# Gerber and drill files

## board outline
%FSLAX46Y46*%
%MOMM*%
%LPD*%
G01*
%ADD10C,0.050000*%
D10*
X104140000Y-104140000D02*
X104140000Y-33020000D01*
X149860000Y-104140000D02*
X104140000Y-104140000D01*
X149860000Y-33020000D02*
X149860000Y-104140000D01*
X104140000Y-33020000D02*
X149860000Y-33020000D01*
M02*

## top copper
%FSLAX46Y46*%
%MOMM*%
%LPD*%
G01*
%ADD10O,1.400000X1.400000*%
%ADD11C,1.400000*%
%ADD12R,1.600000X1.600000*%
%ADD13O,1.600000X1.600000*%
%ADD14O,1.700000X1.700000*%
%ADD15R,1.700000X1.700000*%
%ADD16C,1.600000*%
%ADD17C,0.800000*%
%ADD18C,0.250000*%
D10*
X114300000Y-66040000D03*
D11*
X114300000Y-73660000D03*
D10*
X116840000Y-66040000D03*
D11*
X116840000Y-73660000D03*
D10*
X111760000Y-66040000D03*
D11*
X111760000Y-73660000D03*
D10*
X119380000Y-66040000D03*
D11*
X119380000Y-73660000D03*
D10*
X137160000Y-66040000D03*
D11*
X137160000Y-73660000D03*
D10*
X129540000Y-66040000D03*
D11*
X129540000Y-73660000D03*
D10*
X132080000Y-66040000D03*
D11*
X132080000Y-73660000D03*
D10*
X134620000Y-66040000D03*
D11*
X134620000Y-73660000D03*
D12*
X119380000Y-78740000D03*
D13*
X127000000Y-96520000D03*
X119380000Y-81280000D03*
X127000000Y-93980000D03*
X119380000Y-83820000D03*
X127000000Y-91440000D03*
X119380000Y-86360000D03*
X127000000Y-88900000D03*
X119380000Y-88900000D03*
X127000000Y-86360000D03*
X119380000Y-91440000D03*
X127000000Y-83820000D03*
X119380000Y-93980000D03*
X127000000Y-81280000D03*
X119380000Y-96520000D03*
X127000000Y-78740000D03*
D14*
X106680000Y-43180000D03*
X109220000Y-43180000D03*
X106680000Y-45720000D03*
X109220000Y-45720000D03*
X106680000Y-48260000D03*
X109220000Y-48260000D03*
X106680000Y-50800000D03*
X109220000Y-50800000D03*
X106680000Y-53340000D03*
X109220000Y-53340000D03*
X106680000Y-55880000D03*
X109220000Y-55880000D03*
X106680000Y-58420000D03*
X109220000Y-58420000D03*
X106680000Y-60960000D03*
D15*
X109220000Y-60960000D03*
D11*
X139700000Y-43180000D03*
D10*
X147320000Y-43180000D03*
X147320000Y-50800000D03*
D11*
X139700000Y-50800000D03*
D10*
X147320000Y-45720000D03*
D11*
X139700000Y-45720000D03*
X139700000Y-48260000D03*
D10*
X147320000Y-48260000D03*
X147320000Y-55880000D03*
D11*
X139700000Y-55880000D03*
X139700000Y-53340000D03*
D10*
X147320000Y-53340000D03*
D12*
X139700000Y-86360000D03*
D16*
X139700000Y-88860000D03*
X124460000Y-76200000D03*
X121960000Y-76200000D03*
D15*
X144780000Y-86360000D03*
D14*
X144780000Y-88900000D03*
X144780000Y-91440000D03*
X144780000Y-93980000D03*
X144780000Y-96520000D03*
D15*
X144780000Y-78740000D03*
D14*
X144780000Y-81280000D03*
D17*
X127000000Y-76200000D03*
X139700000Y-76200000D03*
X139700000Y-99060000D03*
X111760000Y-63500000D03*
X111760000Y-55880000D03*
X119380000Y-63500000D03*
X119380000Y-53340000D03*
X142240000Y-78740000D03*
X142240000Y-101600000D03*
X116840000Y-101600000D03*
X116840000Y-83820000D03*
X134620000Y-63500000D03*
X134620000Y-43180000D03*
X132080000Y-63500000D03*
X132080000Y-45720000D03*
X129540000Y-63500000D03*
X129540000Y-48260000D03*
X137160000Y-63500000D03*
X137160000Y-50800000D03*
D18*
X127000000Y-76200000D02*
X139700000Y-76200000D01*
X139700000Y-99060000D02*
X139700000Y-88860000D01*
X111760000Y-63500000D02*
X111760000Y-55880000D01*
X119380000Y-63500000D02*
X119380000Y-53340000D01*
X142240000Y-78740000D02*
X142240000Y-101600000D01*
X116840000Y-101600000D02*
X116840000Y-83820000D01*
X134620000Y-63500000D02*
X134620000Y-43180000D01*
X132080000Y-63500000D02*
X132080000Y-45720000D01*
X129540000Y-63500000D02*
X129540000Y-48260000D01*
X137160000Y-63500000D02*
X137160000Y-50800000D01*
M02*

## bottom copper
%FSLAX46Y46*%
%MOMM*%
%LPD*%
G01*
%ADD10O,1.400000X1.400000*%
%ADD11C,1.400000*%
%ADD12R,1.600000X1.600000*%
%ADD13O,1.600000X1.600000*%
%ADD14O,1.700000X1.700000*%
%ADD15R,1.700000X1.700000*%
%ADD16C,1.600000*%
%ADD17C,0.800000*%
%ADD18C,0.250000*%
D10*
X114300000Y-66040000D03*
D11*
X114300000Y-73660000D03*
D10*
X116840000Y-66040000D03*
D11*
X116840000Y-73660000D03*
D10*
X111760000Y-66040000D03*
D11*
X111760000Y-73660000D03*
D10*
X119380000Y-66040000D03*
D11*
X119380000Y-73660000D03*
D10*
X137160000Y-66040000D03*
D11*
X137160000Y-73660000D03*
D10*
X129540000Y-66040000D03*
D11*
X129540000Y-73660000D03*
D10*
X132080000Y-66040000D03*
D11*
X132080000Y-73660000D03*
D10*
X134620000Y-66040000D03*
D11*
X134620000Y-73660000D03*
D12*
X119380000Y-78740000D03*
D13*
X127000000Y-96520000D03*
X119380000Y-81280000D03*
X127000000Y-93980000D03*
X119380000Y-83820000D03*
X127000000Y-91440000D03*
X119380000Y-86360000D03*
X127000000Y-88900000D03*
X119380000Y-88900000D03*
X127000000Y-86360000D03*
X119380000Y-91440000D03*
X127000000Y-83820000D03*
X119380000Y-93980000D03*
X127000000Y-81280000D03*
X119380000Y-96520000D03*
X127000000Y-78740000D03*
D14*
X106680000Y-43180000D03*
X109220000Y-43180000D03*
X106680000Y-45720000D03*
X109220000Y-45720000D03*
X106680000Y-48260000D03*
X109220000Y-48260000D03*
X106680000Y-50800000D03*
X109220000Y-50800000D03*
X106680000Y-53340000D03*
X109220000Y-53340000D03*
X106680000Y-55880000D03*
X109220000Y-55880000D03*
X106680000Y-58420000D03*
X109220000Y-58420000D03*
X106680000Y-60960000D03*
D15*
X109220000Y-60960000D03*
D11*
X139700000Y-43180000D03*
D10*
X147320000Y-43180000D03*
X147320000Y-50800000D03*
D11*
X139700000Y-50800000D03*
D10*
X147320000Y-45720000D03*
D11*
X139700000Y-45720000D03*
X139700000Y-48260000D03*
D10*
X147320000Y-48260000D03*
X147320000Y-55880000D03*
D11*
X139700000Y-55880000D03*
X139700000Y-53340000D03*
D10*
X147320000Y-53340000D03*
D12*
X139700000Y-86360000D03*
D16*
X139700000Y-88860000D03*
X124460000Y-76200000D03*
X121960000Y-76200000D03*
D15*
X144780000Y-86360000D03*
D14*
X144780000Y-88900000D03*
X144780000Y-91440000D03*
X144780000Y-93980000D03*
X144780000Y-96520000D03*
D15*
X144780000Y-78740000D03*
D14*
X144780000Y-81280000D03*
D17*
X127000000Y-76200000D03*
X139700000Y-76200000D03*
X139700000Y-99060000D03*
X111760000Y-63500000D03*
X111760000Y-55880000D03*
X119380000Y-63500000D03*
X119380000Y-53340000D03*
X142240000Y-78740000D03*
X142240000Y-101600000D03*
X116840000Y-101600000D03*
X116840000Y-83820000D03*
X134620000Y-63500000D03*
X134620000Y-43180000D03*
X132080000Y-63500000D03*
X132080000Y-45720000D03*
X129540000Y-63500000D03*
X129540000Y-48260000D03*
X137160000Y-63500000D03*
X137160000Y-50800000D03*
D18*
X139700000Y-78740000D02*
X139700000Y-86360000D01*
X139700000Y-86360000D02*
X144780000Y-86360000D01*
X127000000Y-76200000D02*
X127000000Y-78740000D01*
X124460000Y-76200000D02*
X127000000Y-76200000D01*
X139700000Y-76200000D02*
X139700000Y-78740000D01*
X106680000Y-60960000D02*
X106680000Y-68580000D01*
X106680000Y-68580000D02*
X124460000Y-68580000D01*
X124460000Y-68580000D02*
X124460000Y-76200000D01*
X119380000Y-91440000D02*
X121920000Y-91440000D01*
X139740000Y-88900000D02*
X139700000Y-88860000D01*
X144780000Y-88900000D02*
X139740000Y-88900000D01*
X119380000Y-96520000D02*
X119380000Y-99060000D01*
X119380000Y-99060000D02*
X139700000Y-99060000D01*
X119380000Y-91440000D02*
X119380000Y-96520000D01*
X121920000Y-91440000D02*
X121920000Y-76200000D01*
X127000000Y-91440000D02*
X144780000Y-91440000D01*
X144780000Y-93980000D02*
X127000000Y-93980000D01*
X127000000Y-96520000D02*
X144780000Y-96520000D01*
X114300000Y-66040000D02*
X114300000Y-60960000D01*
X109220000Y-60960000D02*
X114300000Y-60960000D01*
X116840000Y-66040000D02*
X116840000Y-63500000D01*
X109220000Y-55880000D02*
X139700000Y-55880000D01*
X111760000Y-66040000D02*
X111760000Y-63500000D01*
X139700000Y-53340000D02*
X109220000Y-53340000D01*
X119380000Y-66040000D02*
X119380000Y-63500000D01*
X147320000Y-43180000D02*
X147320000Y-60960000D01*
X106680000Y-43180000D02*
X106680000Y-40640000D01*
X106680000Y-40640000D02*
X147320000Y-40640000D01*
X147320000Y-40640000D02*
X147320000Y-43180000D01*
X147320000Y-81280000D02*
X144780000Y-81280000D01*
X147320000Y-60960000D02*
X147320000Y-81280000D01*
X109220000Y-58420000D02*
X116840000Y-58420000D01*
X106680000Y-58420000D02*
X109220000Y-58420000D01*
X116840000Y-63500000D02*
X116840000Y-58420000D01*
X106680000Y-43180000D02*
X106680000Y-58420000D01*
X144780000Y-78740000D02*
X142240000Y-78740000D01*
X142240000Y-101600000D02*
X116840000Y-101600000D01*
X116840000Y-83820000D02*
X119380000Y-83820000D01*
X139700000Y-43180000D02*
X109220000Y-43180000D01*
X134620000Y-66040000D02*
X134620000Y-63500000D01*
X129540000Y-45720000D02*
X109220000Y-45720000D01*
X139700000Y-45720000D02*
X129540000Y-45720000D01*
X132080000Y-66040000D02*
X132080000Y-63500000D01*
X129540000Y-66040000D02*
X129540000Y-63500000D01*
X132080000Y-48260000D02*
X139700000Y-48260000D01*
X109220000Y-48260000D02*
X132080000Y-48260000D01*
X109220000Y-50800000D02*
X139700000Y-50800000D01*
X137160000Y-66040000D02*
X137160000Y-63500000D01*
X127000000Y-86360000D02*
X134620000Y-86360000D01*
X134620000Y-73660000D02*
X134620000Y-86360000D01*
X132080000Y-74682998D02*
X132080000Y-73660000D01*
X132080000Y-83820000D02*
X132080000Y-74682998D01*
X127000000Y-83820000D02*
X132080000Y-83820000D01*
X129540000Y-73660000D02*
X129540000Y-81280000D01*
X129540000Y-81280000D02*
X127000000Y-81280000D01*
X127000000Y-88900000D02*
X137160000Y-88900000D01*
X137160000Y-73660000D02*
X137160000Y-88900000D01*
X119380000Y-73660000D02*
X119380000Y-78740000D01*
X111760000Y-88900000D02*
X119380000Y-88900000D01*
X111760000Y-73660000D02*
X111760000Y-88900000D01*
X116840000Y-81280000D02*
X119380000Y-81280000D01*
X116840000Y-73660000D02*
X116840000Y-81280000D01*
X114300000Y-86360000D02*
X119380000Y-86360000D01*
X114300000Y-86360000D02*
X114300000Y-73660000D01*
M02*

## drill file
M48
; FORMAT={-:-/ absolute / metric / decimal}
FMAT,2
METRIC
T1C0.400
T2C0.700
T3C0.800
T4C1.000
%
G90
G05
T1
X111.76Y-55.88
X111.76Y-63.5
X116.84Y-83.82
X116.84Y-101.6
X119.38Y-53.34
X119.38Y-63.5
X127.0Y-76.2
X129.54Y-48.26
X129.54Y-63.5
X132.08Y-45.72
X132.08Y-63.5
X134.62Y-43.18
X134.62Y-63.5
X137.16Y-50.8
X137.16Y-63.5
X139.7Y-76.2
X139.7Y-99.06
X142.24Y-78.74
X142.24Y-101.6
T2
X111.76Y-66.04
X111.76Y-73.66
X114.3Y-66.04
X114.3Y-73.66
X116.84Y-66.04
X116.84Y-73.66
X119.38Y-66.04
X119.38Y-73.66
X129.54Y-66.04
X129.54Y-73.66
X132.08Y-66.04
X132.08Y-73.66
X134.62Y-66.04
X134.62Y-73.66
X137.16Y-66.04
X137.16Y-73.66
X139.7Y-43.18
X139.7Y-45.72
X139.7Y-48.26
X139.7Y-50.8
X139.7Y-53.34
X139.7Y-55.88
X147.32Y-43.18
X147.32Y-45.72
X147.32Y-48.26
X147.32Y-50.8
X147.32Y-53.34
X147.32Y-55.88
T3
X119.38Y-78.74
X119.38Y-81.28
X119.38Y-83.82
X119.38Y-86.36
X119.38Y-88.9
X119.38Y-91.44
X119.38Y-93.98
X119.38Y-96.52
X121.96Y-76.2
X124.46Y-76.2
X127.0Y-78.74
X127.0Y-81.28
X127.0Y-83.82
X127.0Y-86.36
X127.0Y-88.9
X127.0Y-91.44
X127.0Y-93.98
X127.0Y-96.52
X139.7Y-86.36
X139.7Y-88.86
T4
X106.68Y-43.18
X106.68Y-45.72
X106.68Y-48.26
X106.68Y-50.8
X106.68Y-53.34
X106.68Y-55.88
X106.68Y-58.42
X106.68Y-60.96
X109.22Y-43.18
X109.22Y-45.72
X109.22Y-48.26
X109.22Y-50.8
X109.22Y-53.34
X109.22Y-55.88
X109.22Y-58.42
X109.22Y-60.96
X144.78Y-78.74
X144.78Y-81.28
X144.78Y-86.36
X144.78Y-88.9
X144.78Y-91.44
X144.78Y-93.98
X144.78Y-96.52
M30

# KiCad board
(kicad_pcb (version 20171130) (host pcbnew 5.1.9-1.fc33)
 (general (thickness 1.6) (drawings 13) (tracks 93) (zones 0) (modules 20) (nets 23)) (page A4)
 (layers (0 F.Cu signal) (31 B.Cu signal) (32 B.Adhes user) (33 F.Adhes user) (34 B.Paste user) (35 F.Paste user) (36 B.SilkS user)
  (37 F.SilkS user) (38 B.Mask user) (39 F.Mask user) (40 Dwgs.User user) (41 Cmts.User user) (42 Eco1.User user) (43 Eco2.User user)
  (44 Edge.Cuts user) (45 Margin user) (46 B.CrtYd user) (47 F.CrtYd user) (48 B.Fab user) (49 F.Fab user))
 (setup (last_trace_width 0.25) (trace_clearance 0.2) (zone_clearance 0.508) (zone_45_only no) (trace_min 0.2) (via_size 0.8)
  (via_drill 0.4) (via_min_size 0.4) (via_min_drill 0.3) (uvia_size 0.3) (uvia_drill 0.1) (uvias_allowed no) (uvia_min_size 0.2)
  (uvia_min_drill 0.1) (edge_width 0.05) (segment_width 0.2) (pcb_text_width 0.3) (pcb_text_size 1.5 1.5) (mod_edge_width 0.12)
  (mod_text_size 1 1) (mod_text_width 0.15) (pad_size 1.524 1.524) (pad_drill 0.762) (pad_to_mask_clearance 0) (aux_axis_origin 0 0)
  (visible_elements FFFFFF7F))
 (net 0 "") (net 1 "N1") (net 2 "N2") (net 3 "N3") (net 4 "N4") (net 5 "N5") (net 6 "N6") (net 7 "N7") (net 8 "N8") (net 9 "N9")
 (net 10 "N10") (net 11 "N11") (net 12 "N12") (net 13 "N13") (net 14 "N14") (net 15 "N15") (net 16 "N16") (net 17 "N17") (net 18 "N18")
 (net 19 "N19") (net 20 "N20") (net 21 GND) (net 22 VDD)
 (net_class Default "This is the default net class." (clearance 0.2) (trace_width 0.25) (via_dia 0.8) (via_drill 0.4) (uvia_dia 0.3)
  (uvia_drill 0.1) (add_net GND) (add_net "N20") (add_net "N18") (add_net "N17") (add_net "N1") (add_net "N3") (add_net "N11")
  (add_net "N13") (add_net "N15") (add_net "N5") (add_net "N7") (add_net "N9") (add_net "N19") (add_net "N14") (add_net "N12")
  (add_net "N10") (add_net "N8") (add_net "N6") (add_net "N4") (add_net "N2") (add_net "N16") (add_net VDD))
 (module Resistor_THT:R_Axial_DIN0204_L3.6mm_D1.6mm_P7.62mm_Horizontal (layer F.Cu) (at 114.3 73.66 90)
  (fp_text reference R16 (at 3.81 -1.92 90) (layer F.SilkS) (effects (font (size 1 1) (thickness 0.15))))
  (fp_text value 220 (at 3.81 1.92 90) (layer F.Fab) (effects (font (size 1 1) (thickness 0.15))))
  (pad 2 thru_hole oval (at 7.62 0 90) (size 1.4 1.4) (drill 0.7) (layers *.Cu *.Mask) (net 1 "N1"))
  (pad 1 thru_hole circle (at 0 0 90) (size 1.4 1.4) (drill 0.7) (layers *.Cu *.Mask) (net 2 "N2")))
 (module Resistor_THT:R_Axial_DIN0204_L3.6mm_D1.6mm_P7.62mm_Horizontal (layer F.Cu) (at 116.84 73.66 90)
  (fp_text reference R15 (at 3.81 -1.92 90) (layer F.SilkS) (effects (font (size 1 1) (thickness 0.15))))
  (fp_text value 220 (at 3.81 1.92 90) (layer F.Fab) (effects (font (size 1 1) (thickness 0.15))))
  (pad 2 thru_hole oval (at 7.62 0 90) (size 1.4 1.4) (drill 0.7) (layers *.Cu *.Mask) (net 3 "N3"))
  (pad 1 thru_hole circle (at 0 0 90) (size 1.4 1.4) (drill 0.7) (layers *.Cu *.Mask) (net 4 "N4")))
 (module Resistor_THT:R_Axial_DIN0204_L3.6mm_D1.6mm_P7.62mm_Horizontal (layer F.Cu) (at 111.76 73.66 90)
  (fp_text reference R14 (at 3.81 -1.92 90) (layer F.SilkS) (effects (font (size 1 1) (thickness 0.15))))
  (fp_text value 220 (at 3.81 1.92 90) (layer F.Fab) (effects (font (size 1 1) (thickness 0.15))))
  (pad 2 thru_hole oval (at 7.62 0 90) (size 1.4 1.4) (drill 0.7) (layers *.Cu *.Mask) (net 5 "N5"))
  (pad 1 thru_hole circle (at 0 0 90) (size 1.4 1.4) (drill 0.7) (layers *.Cu *.Mask) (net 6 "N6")))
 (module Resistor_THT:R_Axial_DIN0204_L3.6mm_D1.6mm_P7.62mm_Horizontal (layer F.Cu) (at 119.38 73.66 90)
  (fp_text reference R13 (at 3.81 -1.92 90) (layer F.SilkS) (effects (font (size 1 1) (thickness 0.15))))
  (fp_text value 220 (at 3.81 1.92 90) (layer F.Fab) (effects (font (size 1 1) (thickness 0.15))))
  (pad 2 thru_hole oval (at 7.62 0 90) (size 1.4 1.4) (drill 0.7) (layers *.Cu *.Mask) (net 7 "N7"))
  (pad 1 thru_hole circle (at 0 0 90) (size 1.4 1.4) (drill 0.7) (layers *.Cu *.Mask) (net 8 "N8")))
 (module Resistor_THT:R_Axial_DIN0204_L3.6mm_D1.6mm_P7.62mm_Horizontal (layer F.Cu) (at 137.16 73.66 90)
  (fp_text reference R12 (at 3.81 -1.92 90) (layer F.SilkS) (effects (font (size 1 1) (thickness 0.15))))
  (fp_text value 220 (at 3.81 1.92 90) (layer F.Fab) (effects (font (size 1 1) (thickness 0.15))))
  (pad 2 thru_hole oval (at 7.62 0 90) (size 1.4 1.4) (drill 0.7) (layers *.Cu *.Mask) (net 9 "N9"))
  (pad 1 thru_hole circle (at 0 0 90) (size 1.4 1.4) (drill 0.7) (layers *.Cu *.Mask) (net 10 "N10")))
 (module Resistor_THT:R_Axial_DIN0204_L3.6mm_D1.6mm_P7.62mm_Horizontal (layer F.Cu) (at 129.54 73.66 90)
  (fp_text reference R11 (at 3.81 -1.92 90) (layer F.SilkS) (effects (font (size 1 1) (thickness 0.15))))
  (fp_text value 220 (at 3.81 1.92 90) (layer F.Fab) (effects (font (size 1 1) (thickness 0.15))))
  (pad 2 thru_hole oval (at 7.62 0 90) (size 1.4 1.4) (drill 0.7) (layers *.Cu *.Mask) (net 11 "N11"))
  (pad 1 thru_hole circle (at 0 0 90) (size 1.4 1.4) (drill 0.7) (layers *.Cu *.Mask) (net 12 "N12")))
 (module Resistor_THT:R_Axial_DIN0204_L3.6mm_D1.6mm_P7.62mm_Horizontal (layer F.Cu) (at 132.08 73.66 90)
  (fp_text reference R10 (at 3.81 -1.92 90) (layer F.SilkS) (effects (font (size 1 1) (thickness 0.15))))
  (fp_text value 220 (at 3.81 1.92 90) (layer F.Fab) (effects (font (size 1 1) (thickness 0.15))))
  (pad 2 thru_hole oval (at 7.62 0 90) (size 1.4 1.4) (drill 0.7) (layers *.Cu *.Mask) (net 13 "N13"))
  (pad 1 thru_hole circle (at 0 0 90) (size 1.4 1.4) (drill 0.7) (layers *.Cu *.Mask) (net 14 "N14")))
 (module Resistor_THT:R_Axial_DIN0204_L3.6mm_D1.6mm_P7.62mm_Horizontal (layer F.Cu) (at 134.62 73.66 90)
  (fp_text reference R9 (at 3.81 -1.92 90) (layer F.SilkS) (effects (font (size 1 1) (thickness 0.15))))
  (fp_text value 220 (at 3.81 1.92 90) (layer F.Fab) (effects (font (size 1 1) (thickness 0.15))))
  (pad 2 thru_hole oval (at 7.62 0 90) (size 1.4 1.4) (drill 0.7) (layers *.Cu *.Mask) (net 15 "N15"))
  (pad 1 thru_hole circle (at 0 0 90) (size 1.4 1.4) (drill 0.7) (layers *.Cu *.Mask) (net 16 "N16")))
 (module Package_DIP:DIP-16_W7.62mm (layer F.Cu) (at 119.38 78.74)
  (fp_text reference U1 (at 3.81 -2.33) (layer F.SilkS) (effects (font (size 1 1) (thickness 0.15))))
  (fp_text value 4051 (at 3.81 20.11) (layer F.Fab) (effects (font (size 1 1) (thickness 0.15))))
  (pad 1 thru_hole rect (at 0 0) (size 1.6 1.6) (drill 0.8) (layers *.Cu *.Mask) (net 8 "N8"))
  (pad 9 thru_hole oval (at 7.62 17.78) (size 1.6 1.6) (drill 0.8) (layers *.Cu *.Mask) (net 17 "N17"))
  (pad 2 thru_hole oval (at 0 2.54) (size 1.6 1.6) (drill 0.8) (layers *.Cu *.Mask) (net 4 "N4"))
  (pad 10 thru_hole oval (at 7.62 15.24) (size 1.6 1.6) (drill 0.8) (layers *.Cu *.Mask) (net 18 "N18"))
  (pad 3 thru_hole oval (at 0 5.08) (size 1.6 1.6) (drill 0.8) (layers *.Cu *.Mask) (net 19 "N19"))
  (pad 11 thru_hole oval (at 7.62 12.7) (size 1.6 1.6) (drill 0.8) (layers *.Cu *.Mask) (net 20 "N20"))
  (pad 4 thru_hole oval (at 0 7.62) (size 1.6 1.6) (drill 0.8) (layers *.Cu *.Mask) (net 2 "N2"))
  (pad 12 thru_hole oval (at 7.62 10.16) (size 1.6 1.6) (drill 0.8) (layers *.Cu *.Mask) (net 10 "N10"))
  (pad 5 thru_hole oval (at 0 10.16) (size 1.6 1.6) (drill 0.8) (layers *.Cu *.Mask) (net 6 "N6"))
  (pad 13 thru_hole oval (at 7.62 7.62) (size 1.6 1.6) (drill 0.8) (layers *.Cu *.Mask) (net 16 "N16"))
  (pad 6 thru_hole oval (at 0 12.7) (size 1.6 1.6) (drill 0.8) (layers *.Cu *.Mask) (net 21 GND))
  (pad 14 thru_hole oval (at 7.62 5.08) (size 1.6 1.6) (drill 0.8) (layers *.Cu *.Mask) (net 14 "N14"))
  (pad 7 thru_hole oval (at 0 15.24) (size 1.6 1.6) (drill 0.8) (layers *.Cu *.Mask) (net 21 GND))
  (pad 15 thru_hole oval (at 7.62 2.54) (size 1.6 1.6) (drill 0.8) (layers *.Cu *.Mask) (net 12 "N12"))
  (pad 8 thru_hole oval (at 0 17.78) (size 1.6 1.6) (drill 0.8) (layers *.Cu *.Mask) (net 21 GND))
  (pad 16 thru_hole oval (at 7.62 0) (size 1.6 1.6) (drill 0.8) (layers *.Cu *.Mask) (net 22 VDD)))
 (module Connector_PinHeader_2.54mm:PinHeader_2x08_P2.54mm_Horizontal (layer F.Cu) (at 109.22 60.96 180)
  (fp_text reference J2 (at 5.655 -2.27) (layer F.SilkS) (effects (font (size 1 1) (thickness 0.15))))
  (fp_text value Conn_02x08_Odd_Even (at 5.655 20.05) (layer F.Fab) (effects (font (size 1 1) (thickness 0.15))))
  (pad 16 thru_hole oval (at 2.54 17.78 180) (size 1.7 1.7) (drill 1) (layers *.Cu *.Mask) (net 3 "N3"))
  (pad 15 thru_hole oval (at 0 17.78 180) (size 1.7 1.7) (drill 1) (layers *.Cu *.Mask) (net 15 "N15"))
  (pad 14 thru_hole oval (at 2.54 15.24 180) (size 1.7 1.7) (drill 1) (layers *.Cu *.Mask) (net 3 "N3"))
  (pad 13 thru_hole oval (at 0 15.24 180) (size 1.7 1.7) (drill 1) (layers *.Cu *.Mask) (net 13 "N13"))
  (pad 12 thru_hole oval (at 2.54 12.7 180) (size 1.7 1.7) (drill 1) (layers *.Cu *.Mask) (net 3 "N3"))
  (pad 11 thru_hole oval (at 0 12.7 180) (size 1.7 1.7) (drill 1) (layers *.Cu *.Mask) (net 11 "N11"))
  (pad 10 thru_hole oval (at 2.54 10.16 180) (size 1.7 1.7) (drill 1) (layers *.Cu *.Mask) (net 3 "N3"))
  (pad 9 thru_hole oval (at 0 10.16 180) (size 1.7 1.7) (drill 1) (layers *.Cu *.Mask) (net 9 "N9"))
  (pad 8 thru_hole oval (at 2.54 7.62 180) (size 1.7 1.7) (drill 1) (layers *.Cu *.Mask) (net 3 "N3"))
  (pad 7 thru_hole oval (at 0 7.62 180) (size 1.7 1.7) (drill 1) (layers *.Cu *.Mask) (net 7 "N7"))
  (pad 6 thru_hole oval (at 2.54 5.08 180) (size 1.7 1.7) (drill 1) (layers *.Cu *.Mask) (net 3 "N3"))
  (pad 5 thru_hole oval (at 0 5.08 180) (size 1.7 1.7) (drill 1) (layers *.Cu *.Mask) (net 5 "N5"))
  (pad 4 thru_hole oval (at 2.54 2.54 180) (size 1.7 1.7) (drill 1) (layers *.Cu *.Mask) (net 3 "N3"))
  (pad 3 thru_hole oval (at 0 2.54 180) (size 1.7 1.7) (drill 1) (layers *.Cu *.Mask) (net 3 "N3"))
  (pad 2 thru_hole oval (at 2.54 0 180) (size 1.7 1.7) (drill 1) (layers *.Cu *.Mask) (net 22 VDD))
  (pad 1 thru_hole rect (at 0 0 180) (size 1.7 1.7) (drill 1) (layers *.Cu *.Mask) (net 1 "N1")))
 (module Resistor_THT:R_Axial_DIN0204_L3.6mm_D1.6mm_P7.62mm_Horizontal (layer F.Cu) (at 139.7 43.18)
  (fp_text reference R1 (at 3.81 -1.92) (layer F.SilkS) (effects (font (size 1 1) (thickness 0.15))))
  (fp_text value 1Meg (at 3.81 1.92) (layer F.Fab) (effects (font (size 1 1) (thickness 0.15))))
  (pad 1 thru_hole circle (at 0 0) (size 1.4 1.4) (drill 0.7) (layers *.Cu *.Mask) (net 15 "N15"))
  (pad 2 thru_hole oval (at 7.62 0) (size 1.4 1.4) (drill 0.7) (layers *.Cu *.Mask) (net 3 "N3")))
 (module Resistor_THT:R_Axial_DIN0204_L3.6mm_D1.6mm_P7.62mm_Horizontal (layer F.Cu) (at 139.7 50.8)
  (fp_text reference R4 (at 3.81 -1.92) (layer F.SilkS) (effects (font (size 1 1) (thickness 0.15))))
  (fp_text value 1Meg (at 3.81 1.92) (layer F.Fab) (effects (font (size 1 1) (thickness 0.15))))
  (pad 2 thru_hole oval (at 7.62 0) (size 1.4 1.4) (drill 0.7) (layers *.Cu *.Mask) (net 3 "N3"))
  (pad 1 thru_hole circle (at 0 0) (size 1.4 1.4) (drill 0.7) (layers *.Cu *.Mask) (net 9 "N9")))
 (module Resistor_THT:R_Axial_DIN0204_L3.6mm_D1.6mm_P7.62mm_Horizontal (layer F.Cu) (at 139.7 45.72)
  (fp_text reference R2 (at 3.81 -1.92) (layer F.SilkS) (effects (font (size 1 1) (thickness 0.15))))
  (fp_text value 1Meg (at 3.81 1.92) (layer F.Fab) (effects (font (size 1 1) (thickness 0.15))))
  (pad 2 thru_hole oval (at 7.62 0) (size 1.4 1.4) (drill 0.7) (layers *.Cu *.Mask) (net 3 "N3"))
  (pad 1 thru_hole circle (at 0 0) (size 1.4 1.4) (drill 0.7) (layers *.Cu *.Mask) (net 13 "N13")))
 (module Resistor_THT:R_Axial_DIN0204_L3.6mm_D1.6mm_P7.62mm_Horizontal (layer F.Cu) (at 139.7 48.26)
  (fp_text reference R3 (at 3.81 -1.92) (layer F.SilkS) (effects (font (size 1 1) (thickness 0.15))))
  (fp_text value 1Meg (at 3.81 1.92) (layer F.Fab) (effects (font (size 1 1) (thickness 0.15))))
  (pad 1 thru_hole circle (at 0 0) (size 1.4 1.4) (drill 0.7) (layers *.Cu *.Mask) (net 11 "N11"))
  (pad 2 thru_hole oval (at 7.62 0) (size 1.4 1.4) (drill 0.7) (layers *.Cu *.Mask) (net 3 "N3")))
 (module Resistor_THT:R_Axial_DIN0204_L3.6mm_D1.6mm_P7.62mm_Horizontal (layer F.Cu) (at 139.7 55.88)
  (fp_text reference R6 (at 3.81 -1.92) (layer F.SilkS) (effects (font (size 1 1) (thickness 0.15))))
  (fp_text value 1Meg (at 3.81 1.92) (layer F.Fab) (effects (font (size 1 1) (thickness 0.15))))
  (pad 2 thru_hole oval (at 7.62 0) (size 1.4 1.4) (drill 0.7) (layers *.Cu *.Mask) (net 3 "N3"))
  (pad 1 thru_hole circle (at 0 0) (size 1.4 1.4) (drill 0.7) (layers *.Cu *.Mask) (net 5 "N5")))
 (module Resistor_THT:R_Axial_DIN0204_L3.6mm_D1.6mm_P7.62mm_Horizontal (layer F.Cu) (at 139.7 53.34)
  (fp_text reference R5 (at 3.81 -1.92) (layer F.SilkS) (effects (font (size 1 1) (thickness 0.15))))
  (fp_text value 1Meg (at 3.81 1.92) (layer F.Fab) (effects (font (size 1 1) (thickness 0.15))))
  (pad 1 thru_hole circle (at 0 0) (size 1.4 1.4) (drill 0.7) (layers *.Cu *.Mask) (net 7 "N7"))
  (pad 2 thru_hole oval (at 7.62 0) (size 1.4 1.4) (drill 0.7) (layers *.Cu *.Mask) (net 3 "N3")))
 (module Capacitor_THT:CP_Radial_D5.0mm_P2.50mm (layer F.Cu) (at 139.7 86.36 270)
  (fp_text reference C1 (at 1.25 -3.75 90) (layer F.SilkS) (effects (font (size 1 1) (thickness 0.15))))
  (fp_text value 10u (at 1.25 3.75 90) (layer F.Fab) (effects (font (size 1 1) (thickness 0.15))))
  (pad 1 thru_hole rect (at 0 0 270) (size 1.6 1.6) (drill 0.8) (layers *.Cu *.Mask) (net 22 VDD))
  (pad 2 thru_hole circle (at 2.5 0 270) (size 1.6 1.6) (drill 0.8) (layers *.Cu *.Mask) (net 21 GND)))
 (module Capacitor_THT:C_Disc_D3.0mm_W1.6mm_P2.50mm (layer F.Cu) (at 124.46 76.2 180)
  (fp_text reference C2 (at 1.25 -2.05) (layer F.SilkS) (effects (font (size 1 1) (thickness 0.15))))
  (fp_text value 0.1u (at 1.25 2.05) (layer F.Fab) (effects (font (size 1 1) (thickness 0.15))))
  (pad 1 thru_hole circle (at 0 0 180) (size 1.6 1.6) (drill 0.8) (layers *.Cu *.Mask) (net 22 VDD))
  (pad 2 thru_hole circle (at 2.5 0 180) (size 1.6 1.6) (drill 0.8) (layers *.Cu *.Mask) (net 21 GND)))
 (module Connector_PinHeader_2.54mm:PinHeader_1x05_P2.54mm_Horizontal (layer F.Cu) (at 144.78 86.36)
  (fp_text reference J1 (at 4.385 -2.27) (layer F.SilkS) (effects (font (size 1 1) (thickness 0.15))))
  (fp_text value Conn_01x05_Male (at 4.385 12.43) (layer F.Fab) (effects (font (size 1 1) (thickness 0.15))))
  (pad 1 thru_hole rect (at 0 0) (size 1.7 1.7) (drill 1) (layers *.Cu *.Mask) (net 22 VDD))
  (pad 2 thru_hole oval (at 0 2.54) (size 1.7 1.7) (drill 1) (layers *.Cu *.Mask) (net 21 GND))
  (pad 3 thru_hole oval (at 0 5.08) (size 1.7 1.7) (drill 1) (layers *.Cu *.Mask) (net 20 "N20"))
  (pad 4 thru_hole oval (at 0 7.62) (size 1.7 1.7) (drill 1) (layers *.Cu *.Mask) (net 18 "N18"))
  (pad 5 thru_hole oval (at 0 10.16) (size 1.7 1.7) (drill 1) (layers *.Cu *.Mask) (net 17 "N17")))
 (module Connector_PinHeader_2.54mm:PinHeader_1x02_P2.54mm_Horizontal (layer F.Cu) (at 144.78 78.74)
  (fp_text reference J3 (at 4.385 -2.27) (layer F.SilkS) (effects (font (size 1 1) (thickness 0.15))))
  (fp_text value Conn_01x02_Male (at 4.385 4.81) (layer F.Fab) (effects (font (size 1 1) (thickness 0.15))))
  (pad 1 thru_hole rect (at 0 0) (size 1.7 1.7) (drill 1) (layers *.Cu *.Mask) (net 19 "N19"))
  (pad 2 thru_hole oval (at 0 2.54) (size 1.7 1.7) (drill 1) (layers *.Cu *.Mask) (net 3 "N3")))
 (gr_line (start 104.14 104.14) (end 104.14 33.02) (layer Edge.Cuts) (width 0.05))
 (gr_line (start 149.86 104.14) (end 104.14 104.14) (layer Edge.Cuts) (width 0.05))
 (gr_line (start 149.86 33.02) (end 149.86 104.14) (layer Edge.Cuts) (width 0.05))
 (gr_line (start 104.14 33.02) (end 149.86 33.02) (layer Edge.Cuts) (width 0.05))
 (segment (start 139.7 78.74) (end 139.7 86.36) (width 0.25) (layer B.Cu) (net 22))
 (segment (start 139.7 86.36) (end 144.78 86.36) (width 0.25) (layer B.Cu) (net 22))
 (segment (start 127 76.2) (end 127 78.74) (width 0.25) (layer B.Cu) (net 22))
 (via (at 127 76.2) (size 0.8) (drill 0.4) (layers F.Cu B.Cu) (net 22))
 (segment (start 124.46 76.2) (end 127 76.2) (width 0.25) (layer B.Cu) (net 22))
 (via (at 139.7 76.2) (size 0.8) (drill 0.4) (layers F.Cu B.Cu) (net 22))
 (segment (start 127 76.2) (end 139.7 76.2) (width 0.25) (layer F.Cu) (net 22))
 (segment (start 139.7 76.2) (end 139.7 78.74) (width 0.25) (layer B.Cu) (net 22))
 (segment (start 106.68 60.96) (end 106.68 68.58) (width 0.25) (layer B.Cu) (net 22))
 (segment (start 106.68 68.58) (end 124.46 68.58) (width 0.25) (layer B.Cu) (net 22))
 (segment (start 124.46 68.58) (end 124.46 76.2) (width 0.25) (layer B.Cu) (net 22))
 (segment (start 119.38 91.44) (end 121.92 91.44) (width 0.25) (layer B.Cu) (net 21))
 (segment (start 139.74 88.9) (end 139.7 88.86) (width 0.25) (layer B.Cu) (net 21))
 (segment (start 144.78 88.9) (end 139.74 88.9) (width 0.25) (layer B.Cu) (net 21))
 (segment (start 119.38 96.52) (end 119.38 99.06) (width 0.25) (layer B.Cu) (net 21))
 (via (at 139.7 99.06) (size 0.8) (drill 0.4) (layers F.Cu B.Cu) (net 21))
 (segment (start 119.38 99.06) (end 139.7 99.06) (width 0.25) (layer B.Cu) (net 21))
 (segment (start 139.7 99.06) (end 139.7 88.86) (width 0.25) (layer F.Cu) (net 21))
 (segment (start 119.38 91.44) (end 119.38 96.52) (width 0.25) (layer B.Cu) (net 21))
 (segment (start 121.92 91.44) (end 121.92 76.2) (width 0.25) (layer B.Cu) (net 21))
 (segment (start 127 91.44) (end 144.78 91.44) (width 0.25) (layer B.Cu) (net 20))
 (segment (start 144.78 93.98) (end 127 93.98) (width 0.25) (layer B.Cu) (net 18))
 (segment (start 127 96.52) (end 144.78 96.52) (width 0.25) (layer B.Cu) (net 17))
 (segment (start 114.3 66.04) (end 114.3 60.96) (width 0.25) (layer B.Cu) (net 1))
 (segment (start 109.22 60.96) (end 114.3 60.96) (width 0.25) (layer B.Cu) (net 1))
 (segment (start 116.84 66.04) (end 116.84 63.5) (width 0.25) (layer B.Cu) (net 3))
 (segment (start 109.22 55.88) (end 139.7 55.88) (width 0.25) (layer B.Cu) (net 5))
 (via (at 111.76 63.5) (size 0.8) (drill 0.4) (layers F.Cu B.Cu) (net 5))
 (segment (start 111.76 66.04) (end 111.76 63.5) (width 0.25) (layer B.Cu) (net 5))
 (segment (start 111.76 63.5) (end 111.76 55.88) (width 0.25) (layer F.Cu) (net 5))
 (via (at 111.76 55.88) (size 0.8) (drill 0.4) (layers F.Cu B.Cu) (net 5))
 (segment (start 139.7 53.34) (end 109.22 53.34) (width 0.25) (layer B.Cu) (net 7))
 (via (at 119.38 63.5) (size 0.8) (drill 0.4) (layers F.Cu B.Cu) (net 7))
 (segment (start 119.38 66.04) (end 119.38 63.5) (width 0.25) (layer B.Cu) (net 7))
 (via (at 119.38 53.34) (size 0.8) (drill 0.4) (layers F.Cu B.Cu) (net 7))
 (segment (start 119.38 63.5) (end 119.38 53.34) (width 0.25) (layer F.Cu) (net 7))
 (segment (start 147.32 43.18) (end 147.32 60.96) (width 0.25) (layer B.Cu) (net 3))
 (segment (start 106.68 43.18) (end 106.68 40.64) (width 0.25) (layer B.Cu) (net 3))
 (segment (start 106.68 40.64) (end 147.32 40.64) (width 0.25) (layer B.Cu) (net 3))
 (segment (start 147.32 40.64) (end 147.32 43.18) (width 0.25) (layer B.Cu) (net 3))
 (segment (start 147.32 81.28) (end 144.78 81.28) (width 0.25) (layer B.Cu) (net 3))
 (segment (start 147.32 60.96) (end 147.32 81.28) (width 0.25) (layer B.Cu) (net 3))
 (segment (start 109.22 58.42) (end 116.84 58.42) (width 0.25) (layer B.Cu) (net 3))
 (segment (start 106.68 58.42) (end 109.22 58.42) (width 0.25) (layer B.Cu) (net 3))
 (segment (start 116.84 63.5) (end 116.84 58.42) (width 0.25) (layer B.Cu) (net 3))
 (segment (start 106.68 43.18) (end 106.68 58.42) (width 0.25) (layer B.Cu) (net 3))
 (via (at 142.24 78.74) (size 0.8) (drill 0.4) (layers F.Cu B.Cu) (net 19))
 (segment (start 144.78 78.74) (end 142.24 78.74) (width 0.25) (layer B.Cu) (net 19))
 (via (at 142.24 101.6) (size 0.8) (drill 0.4) (layers F.Cu B.Cu) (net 19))
 (segment (start 142.24 78.74) (end 142.24 101.6) (width 0.25) (layer F.Cu) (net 19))
 (via (at 116.84 101.6) (size 0.8) (drill 0.4) (layers F.Cu B.Cu) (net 19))
 (segment (start 142.24 101.6) (end 116.84 101.6) (width 0.25) (layer B.Cu) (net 19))
 (via (at 116.84 83.82) (size 0.8) (drill 0.4) (layers F.Cu B.Cu) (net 19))
 (segment (start 116.84 101.6) (end 116.84 83.82) (width 0.25) (layer F.Cu) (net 19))
 (segment (start 116.84 83.82) (end 119.38 83.82) (width 0.25) (layer B.Cu) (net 19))
 (segment (start 139.7 43.18) (end 109.22 43.18) (width 0.25) (layer B.Cu) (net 15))
 (via (at 134.62 63.5) (size 0.8) (drill 0.4) (layers F.Cu B.Cu) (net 15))
 (segment (start 134.62 66.04) (end 134.62 63.5) (width 0.25) (layer B.Cu) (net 15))
 (via (at 134.62 43.18) (size 0.8) (drill 0.4) (layers F.Cu B.Cu) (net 15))
 (segment (start 134.62 63.5) (end 134.62 43.18) (width 0.25) (layer F.Cu) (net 15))
 (segment (start 129.54 45.72) (end 109.22 45.72) (width 0.25) (layer B.Cu) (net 13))
 (segment (start 139.7 45.72) (end 129.54 45.72) (width 0.25) (layer B.Cu) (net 13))
 (via (at 132.08 63.5) (size 0.8) (drill 0.4) (layers F.Cu B.Cu) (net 13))
 (segment (start 132.08 66.04) (end 132.08 63.5) (width 0.25) (layer B.Cu) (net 13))
 (via (at 132.08 45.72) (size 0.8) (drill 0.4) (layers F.Cu B.Cu) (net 13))
 (segment (start 132.08 63.5) (end 132.08 45.72) (width 0.25) (layer F.Cu) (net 13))
 (via (at 129.54 63.5) (size 0.8) (drill 0.4) (layers F.Cu B.Cu) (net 11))
 (segment (start 129.54 66.04) (end 129.54 63.5) (width 0.25) (layer B.Cu) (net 11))
 (segment (start 132.08 48.26) (end 139.7 48.26) (width 0.25) (layer B.Cu) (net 11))
 (segment (start 109.22 48.26) (end 132.08 48.26) (width 0.25) (layer B.Cu) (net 11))
 (via (at 129.54 48.26) (size 0.8) (drill 0.4) (layers F.Cu B.Cu) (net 11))
 (segment (start 129.54 63.5) (end 129.54 48.26) (width 0.25) (layer F.Cu) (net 11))
 (segment (start 109.22 50.8) (end 139.7 50.8) (width 0.25) (layer B.Cu) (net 9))
 (via (at 137.16 63.5) (size 0.8) (drill 0.4) (layers F.Cu B.Cu) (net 9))
 (segment (start 137.16 66.04) (end 137.16 63.5) (width 0.25) (layer B.Cu) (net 9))
 (via (at 137.16 50.8) (size 0.8) (drill 0.4) (layers F.Cu B.Cu) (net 9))
 (segment (start 137.16 63.5) (end 137.16 50.8) (width 0.25) (layer F.Cu) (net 9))
 (segment (start 127 86.36) (end 134.62 86.36) (width 0.25) (layer B.Cu) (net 16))
 (segment (start 134.62 73.66) (end 134.62 86.36) (width 0.25) (layer B.Cu) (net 16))
 (segment (start 132.08 74.682998) (end 132.08 73.66) (width 0.25) (layer B.Cu) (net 14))
 (segment (start 132.08 83.82) (end 132.08 74.682998) (width 0.25) (layer B.Cu) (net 14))
 (segment (start 127 83.82) (end 132.08 83.82) (width 0.25) (layer B.Cu) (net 14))
 (segment (start 129.54 73.66) (end 129.54 81.28) (width 0.25) (layer B.Cu) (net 12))
 (segment (start 129.54 81.28) (end 127 81.28) (width 0.25) (layer B.Cu) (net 12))
 (segment (start 127 88.9) (end 137.16 88.9) (width 0.25) (layer B.Cu) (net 10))
 (segment (start 137.16 73.66) (end 137.16 88.9) (width 0.25) (layer B.Cu) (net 10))
 (segment (start 119.38 73.66) (end 119.38 78.74) (width 0.25) (layer B.Cu) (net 8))
 (segment (start 111.76 88.9) (end 119.38 88.9) (width 0.25) (layer B.Cu) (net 6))
 (segment (start 111.76 73.66) (end 111.76 88.9) (width 0.25) (layer B.Cu) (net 6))
 (segment (start 116.84 81.28) (end 119.38 81.28) (width 0.25) (layer B.Cu) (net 4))
 (segment (start 116.84 73.66) (end 116.84 81.28) (width 0.25) (layer B.Cu) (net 4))
 (segment (start 114.3 86.36) (end 119.38 86.36) (width 0.25) (layer B.Cu) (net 2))
 (segment (start 114.3 86.36) (end 114.3 73.66) (width 0.25) (layer B.Cu) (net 2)))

